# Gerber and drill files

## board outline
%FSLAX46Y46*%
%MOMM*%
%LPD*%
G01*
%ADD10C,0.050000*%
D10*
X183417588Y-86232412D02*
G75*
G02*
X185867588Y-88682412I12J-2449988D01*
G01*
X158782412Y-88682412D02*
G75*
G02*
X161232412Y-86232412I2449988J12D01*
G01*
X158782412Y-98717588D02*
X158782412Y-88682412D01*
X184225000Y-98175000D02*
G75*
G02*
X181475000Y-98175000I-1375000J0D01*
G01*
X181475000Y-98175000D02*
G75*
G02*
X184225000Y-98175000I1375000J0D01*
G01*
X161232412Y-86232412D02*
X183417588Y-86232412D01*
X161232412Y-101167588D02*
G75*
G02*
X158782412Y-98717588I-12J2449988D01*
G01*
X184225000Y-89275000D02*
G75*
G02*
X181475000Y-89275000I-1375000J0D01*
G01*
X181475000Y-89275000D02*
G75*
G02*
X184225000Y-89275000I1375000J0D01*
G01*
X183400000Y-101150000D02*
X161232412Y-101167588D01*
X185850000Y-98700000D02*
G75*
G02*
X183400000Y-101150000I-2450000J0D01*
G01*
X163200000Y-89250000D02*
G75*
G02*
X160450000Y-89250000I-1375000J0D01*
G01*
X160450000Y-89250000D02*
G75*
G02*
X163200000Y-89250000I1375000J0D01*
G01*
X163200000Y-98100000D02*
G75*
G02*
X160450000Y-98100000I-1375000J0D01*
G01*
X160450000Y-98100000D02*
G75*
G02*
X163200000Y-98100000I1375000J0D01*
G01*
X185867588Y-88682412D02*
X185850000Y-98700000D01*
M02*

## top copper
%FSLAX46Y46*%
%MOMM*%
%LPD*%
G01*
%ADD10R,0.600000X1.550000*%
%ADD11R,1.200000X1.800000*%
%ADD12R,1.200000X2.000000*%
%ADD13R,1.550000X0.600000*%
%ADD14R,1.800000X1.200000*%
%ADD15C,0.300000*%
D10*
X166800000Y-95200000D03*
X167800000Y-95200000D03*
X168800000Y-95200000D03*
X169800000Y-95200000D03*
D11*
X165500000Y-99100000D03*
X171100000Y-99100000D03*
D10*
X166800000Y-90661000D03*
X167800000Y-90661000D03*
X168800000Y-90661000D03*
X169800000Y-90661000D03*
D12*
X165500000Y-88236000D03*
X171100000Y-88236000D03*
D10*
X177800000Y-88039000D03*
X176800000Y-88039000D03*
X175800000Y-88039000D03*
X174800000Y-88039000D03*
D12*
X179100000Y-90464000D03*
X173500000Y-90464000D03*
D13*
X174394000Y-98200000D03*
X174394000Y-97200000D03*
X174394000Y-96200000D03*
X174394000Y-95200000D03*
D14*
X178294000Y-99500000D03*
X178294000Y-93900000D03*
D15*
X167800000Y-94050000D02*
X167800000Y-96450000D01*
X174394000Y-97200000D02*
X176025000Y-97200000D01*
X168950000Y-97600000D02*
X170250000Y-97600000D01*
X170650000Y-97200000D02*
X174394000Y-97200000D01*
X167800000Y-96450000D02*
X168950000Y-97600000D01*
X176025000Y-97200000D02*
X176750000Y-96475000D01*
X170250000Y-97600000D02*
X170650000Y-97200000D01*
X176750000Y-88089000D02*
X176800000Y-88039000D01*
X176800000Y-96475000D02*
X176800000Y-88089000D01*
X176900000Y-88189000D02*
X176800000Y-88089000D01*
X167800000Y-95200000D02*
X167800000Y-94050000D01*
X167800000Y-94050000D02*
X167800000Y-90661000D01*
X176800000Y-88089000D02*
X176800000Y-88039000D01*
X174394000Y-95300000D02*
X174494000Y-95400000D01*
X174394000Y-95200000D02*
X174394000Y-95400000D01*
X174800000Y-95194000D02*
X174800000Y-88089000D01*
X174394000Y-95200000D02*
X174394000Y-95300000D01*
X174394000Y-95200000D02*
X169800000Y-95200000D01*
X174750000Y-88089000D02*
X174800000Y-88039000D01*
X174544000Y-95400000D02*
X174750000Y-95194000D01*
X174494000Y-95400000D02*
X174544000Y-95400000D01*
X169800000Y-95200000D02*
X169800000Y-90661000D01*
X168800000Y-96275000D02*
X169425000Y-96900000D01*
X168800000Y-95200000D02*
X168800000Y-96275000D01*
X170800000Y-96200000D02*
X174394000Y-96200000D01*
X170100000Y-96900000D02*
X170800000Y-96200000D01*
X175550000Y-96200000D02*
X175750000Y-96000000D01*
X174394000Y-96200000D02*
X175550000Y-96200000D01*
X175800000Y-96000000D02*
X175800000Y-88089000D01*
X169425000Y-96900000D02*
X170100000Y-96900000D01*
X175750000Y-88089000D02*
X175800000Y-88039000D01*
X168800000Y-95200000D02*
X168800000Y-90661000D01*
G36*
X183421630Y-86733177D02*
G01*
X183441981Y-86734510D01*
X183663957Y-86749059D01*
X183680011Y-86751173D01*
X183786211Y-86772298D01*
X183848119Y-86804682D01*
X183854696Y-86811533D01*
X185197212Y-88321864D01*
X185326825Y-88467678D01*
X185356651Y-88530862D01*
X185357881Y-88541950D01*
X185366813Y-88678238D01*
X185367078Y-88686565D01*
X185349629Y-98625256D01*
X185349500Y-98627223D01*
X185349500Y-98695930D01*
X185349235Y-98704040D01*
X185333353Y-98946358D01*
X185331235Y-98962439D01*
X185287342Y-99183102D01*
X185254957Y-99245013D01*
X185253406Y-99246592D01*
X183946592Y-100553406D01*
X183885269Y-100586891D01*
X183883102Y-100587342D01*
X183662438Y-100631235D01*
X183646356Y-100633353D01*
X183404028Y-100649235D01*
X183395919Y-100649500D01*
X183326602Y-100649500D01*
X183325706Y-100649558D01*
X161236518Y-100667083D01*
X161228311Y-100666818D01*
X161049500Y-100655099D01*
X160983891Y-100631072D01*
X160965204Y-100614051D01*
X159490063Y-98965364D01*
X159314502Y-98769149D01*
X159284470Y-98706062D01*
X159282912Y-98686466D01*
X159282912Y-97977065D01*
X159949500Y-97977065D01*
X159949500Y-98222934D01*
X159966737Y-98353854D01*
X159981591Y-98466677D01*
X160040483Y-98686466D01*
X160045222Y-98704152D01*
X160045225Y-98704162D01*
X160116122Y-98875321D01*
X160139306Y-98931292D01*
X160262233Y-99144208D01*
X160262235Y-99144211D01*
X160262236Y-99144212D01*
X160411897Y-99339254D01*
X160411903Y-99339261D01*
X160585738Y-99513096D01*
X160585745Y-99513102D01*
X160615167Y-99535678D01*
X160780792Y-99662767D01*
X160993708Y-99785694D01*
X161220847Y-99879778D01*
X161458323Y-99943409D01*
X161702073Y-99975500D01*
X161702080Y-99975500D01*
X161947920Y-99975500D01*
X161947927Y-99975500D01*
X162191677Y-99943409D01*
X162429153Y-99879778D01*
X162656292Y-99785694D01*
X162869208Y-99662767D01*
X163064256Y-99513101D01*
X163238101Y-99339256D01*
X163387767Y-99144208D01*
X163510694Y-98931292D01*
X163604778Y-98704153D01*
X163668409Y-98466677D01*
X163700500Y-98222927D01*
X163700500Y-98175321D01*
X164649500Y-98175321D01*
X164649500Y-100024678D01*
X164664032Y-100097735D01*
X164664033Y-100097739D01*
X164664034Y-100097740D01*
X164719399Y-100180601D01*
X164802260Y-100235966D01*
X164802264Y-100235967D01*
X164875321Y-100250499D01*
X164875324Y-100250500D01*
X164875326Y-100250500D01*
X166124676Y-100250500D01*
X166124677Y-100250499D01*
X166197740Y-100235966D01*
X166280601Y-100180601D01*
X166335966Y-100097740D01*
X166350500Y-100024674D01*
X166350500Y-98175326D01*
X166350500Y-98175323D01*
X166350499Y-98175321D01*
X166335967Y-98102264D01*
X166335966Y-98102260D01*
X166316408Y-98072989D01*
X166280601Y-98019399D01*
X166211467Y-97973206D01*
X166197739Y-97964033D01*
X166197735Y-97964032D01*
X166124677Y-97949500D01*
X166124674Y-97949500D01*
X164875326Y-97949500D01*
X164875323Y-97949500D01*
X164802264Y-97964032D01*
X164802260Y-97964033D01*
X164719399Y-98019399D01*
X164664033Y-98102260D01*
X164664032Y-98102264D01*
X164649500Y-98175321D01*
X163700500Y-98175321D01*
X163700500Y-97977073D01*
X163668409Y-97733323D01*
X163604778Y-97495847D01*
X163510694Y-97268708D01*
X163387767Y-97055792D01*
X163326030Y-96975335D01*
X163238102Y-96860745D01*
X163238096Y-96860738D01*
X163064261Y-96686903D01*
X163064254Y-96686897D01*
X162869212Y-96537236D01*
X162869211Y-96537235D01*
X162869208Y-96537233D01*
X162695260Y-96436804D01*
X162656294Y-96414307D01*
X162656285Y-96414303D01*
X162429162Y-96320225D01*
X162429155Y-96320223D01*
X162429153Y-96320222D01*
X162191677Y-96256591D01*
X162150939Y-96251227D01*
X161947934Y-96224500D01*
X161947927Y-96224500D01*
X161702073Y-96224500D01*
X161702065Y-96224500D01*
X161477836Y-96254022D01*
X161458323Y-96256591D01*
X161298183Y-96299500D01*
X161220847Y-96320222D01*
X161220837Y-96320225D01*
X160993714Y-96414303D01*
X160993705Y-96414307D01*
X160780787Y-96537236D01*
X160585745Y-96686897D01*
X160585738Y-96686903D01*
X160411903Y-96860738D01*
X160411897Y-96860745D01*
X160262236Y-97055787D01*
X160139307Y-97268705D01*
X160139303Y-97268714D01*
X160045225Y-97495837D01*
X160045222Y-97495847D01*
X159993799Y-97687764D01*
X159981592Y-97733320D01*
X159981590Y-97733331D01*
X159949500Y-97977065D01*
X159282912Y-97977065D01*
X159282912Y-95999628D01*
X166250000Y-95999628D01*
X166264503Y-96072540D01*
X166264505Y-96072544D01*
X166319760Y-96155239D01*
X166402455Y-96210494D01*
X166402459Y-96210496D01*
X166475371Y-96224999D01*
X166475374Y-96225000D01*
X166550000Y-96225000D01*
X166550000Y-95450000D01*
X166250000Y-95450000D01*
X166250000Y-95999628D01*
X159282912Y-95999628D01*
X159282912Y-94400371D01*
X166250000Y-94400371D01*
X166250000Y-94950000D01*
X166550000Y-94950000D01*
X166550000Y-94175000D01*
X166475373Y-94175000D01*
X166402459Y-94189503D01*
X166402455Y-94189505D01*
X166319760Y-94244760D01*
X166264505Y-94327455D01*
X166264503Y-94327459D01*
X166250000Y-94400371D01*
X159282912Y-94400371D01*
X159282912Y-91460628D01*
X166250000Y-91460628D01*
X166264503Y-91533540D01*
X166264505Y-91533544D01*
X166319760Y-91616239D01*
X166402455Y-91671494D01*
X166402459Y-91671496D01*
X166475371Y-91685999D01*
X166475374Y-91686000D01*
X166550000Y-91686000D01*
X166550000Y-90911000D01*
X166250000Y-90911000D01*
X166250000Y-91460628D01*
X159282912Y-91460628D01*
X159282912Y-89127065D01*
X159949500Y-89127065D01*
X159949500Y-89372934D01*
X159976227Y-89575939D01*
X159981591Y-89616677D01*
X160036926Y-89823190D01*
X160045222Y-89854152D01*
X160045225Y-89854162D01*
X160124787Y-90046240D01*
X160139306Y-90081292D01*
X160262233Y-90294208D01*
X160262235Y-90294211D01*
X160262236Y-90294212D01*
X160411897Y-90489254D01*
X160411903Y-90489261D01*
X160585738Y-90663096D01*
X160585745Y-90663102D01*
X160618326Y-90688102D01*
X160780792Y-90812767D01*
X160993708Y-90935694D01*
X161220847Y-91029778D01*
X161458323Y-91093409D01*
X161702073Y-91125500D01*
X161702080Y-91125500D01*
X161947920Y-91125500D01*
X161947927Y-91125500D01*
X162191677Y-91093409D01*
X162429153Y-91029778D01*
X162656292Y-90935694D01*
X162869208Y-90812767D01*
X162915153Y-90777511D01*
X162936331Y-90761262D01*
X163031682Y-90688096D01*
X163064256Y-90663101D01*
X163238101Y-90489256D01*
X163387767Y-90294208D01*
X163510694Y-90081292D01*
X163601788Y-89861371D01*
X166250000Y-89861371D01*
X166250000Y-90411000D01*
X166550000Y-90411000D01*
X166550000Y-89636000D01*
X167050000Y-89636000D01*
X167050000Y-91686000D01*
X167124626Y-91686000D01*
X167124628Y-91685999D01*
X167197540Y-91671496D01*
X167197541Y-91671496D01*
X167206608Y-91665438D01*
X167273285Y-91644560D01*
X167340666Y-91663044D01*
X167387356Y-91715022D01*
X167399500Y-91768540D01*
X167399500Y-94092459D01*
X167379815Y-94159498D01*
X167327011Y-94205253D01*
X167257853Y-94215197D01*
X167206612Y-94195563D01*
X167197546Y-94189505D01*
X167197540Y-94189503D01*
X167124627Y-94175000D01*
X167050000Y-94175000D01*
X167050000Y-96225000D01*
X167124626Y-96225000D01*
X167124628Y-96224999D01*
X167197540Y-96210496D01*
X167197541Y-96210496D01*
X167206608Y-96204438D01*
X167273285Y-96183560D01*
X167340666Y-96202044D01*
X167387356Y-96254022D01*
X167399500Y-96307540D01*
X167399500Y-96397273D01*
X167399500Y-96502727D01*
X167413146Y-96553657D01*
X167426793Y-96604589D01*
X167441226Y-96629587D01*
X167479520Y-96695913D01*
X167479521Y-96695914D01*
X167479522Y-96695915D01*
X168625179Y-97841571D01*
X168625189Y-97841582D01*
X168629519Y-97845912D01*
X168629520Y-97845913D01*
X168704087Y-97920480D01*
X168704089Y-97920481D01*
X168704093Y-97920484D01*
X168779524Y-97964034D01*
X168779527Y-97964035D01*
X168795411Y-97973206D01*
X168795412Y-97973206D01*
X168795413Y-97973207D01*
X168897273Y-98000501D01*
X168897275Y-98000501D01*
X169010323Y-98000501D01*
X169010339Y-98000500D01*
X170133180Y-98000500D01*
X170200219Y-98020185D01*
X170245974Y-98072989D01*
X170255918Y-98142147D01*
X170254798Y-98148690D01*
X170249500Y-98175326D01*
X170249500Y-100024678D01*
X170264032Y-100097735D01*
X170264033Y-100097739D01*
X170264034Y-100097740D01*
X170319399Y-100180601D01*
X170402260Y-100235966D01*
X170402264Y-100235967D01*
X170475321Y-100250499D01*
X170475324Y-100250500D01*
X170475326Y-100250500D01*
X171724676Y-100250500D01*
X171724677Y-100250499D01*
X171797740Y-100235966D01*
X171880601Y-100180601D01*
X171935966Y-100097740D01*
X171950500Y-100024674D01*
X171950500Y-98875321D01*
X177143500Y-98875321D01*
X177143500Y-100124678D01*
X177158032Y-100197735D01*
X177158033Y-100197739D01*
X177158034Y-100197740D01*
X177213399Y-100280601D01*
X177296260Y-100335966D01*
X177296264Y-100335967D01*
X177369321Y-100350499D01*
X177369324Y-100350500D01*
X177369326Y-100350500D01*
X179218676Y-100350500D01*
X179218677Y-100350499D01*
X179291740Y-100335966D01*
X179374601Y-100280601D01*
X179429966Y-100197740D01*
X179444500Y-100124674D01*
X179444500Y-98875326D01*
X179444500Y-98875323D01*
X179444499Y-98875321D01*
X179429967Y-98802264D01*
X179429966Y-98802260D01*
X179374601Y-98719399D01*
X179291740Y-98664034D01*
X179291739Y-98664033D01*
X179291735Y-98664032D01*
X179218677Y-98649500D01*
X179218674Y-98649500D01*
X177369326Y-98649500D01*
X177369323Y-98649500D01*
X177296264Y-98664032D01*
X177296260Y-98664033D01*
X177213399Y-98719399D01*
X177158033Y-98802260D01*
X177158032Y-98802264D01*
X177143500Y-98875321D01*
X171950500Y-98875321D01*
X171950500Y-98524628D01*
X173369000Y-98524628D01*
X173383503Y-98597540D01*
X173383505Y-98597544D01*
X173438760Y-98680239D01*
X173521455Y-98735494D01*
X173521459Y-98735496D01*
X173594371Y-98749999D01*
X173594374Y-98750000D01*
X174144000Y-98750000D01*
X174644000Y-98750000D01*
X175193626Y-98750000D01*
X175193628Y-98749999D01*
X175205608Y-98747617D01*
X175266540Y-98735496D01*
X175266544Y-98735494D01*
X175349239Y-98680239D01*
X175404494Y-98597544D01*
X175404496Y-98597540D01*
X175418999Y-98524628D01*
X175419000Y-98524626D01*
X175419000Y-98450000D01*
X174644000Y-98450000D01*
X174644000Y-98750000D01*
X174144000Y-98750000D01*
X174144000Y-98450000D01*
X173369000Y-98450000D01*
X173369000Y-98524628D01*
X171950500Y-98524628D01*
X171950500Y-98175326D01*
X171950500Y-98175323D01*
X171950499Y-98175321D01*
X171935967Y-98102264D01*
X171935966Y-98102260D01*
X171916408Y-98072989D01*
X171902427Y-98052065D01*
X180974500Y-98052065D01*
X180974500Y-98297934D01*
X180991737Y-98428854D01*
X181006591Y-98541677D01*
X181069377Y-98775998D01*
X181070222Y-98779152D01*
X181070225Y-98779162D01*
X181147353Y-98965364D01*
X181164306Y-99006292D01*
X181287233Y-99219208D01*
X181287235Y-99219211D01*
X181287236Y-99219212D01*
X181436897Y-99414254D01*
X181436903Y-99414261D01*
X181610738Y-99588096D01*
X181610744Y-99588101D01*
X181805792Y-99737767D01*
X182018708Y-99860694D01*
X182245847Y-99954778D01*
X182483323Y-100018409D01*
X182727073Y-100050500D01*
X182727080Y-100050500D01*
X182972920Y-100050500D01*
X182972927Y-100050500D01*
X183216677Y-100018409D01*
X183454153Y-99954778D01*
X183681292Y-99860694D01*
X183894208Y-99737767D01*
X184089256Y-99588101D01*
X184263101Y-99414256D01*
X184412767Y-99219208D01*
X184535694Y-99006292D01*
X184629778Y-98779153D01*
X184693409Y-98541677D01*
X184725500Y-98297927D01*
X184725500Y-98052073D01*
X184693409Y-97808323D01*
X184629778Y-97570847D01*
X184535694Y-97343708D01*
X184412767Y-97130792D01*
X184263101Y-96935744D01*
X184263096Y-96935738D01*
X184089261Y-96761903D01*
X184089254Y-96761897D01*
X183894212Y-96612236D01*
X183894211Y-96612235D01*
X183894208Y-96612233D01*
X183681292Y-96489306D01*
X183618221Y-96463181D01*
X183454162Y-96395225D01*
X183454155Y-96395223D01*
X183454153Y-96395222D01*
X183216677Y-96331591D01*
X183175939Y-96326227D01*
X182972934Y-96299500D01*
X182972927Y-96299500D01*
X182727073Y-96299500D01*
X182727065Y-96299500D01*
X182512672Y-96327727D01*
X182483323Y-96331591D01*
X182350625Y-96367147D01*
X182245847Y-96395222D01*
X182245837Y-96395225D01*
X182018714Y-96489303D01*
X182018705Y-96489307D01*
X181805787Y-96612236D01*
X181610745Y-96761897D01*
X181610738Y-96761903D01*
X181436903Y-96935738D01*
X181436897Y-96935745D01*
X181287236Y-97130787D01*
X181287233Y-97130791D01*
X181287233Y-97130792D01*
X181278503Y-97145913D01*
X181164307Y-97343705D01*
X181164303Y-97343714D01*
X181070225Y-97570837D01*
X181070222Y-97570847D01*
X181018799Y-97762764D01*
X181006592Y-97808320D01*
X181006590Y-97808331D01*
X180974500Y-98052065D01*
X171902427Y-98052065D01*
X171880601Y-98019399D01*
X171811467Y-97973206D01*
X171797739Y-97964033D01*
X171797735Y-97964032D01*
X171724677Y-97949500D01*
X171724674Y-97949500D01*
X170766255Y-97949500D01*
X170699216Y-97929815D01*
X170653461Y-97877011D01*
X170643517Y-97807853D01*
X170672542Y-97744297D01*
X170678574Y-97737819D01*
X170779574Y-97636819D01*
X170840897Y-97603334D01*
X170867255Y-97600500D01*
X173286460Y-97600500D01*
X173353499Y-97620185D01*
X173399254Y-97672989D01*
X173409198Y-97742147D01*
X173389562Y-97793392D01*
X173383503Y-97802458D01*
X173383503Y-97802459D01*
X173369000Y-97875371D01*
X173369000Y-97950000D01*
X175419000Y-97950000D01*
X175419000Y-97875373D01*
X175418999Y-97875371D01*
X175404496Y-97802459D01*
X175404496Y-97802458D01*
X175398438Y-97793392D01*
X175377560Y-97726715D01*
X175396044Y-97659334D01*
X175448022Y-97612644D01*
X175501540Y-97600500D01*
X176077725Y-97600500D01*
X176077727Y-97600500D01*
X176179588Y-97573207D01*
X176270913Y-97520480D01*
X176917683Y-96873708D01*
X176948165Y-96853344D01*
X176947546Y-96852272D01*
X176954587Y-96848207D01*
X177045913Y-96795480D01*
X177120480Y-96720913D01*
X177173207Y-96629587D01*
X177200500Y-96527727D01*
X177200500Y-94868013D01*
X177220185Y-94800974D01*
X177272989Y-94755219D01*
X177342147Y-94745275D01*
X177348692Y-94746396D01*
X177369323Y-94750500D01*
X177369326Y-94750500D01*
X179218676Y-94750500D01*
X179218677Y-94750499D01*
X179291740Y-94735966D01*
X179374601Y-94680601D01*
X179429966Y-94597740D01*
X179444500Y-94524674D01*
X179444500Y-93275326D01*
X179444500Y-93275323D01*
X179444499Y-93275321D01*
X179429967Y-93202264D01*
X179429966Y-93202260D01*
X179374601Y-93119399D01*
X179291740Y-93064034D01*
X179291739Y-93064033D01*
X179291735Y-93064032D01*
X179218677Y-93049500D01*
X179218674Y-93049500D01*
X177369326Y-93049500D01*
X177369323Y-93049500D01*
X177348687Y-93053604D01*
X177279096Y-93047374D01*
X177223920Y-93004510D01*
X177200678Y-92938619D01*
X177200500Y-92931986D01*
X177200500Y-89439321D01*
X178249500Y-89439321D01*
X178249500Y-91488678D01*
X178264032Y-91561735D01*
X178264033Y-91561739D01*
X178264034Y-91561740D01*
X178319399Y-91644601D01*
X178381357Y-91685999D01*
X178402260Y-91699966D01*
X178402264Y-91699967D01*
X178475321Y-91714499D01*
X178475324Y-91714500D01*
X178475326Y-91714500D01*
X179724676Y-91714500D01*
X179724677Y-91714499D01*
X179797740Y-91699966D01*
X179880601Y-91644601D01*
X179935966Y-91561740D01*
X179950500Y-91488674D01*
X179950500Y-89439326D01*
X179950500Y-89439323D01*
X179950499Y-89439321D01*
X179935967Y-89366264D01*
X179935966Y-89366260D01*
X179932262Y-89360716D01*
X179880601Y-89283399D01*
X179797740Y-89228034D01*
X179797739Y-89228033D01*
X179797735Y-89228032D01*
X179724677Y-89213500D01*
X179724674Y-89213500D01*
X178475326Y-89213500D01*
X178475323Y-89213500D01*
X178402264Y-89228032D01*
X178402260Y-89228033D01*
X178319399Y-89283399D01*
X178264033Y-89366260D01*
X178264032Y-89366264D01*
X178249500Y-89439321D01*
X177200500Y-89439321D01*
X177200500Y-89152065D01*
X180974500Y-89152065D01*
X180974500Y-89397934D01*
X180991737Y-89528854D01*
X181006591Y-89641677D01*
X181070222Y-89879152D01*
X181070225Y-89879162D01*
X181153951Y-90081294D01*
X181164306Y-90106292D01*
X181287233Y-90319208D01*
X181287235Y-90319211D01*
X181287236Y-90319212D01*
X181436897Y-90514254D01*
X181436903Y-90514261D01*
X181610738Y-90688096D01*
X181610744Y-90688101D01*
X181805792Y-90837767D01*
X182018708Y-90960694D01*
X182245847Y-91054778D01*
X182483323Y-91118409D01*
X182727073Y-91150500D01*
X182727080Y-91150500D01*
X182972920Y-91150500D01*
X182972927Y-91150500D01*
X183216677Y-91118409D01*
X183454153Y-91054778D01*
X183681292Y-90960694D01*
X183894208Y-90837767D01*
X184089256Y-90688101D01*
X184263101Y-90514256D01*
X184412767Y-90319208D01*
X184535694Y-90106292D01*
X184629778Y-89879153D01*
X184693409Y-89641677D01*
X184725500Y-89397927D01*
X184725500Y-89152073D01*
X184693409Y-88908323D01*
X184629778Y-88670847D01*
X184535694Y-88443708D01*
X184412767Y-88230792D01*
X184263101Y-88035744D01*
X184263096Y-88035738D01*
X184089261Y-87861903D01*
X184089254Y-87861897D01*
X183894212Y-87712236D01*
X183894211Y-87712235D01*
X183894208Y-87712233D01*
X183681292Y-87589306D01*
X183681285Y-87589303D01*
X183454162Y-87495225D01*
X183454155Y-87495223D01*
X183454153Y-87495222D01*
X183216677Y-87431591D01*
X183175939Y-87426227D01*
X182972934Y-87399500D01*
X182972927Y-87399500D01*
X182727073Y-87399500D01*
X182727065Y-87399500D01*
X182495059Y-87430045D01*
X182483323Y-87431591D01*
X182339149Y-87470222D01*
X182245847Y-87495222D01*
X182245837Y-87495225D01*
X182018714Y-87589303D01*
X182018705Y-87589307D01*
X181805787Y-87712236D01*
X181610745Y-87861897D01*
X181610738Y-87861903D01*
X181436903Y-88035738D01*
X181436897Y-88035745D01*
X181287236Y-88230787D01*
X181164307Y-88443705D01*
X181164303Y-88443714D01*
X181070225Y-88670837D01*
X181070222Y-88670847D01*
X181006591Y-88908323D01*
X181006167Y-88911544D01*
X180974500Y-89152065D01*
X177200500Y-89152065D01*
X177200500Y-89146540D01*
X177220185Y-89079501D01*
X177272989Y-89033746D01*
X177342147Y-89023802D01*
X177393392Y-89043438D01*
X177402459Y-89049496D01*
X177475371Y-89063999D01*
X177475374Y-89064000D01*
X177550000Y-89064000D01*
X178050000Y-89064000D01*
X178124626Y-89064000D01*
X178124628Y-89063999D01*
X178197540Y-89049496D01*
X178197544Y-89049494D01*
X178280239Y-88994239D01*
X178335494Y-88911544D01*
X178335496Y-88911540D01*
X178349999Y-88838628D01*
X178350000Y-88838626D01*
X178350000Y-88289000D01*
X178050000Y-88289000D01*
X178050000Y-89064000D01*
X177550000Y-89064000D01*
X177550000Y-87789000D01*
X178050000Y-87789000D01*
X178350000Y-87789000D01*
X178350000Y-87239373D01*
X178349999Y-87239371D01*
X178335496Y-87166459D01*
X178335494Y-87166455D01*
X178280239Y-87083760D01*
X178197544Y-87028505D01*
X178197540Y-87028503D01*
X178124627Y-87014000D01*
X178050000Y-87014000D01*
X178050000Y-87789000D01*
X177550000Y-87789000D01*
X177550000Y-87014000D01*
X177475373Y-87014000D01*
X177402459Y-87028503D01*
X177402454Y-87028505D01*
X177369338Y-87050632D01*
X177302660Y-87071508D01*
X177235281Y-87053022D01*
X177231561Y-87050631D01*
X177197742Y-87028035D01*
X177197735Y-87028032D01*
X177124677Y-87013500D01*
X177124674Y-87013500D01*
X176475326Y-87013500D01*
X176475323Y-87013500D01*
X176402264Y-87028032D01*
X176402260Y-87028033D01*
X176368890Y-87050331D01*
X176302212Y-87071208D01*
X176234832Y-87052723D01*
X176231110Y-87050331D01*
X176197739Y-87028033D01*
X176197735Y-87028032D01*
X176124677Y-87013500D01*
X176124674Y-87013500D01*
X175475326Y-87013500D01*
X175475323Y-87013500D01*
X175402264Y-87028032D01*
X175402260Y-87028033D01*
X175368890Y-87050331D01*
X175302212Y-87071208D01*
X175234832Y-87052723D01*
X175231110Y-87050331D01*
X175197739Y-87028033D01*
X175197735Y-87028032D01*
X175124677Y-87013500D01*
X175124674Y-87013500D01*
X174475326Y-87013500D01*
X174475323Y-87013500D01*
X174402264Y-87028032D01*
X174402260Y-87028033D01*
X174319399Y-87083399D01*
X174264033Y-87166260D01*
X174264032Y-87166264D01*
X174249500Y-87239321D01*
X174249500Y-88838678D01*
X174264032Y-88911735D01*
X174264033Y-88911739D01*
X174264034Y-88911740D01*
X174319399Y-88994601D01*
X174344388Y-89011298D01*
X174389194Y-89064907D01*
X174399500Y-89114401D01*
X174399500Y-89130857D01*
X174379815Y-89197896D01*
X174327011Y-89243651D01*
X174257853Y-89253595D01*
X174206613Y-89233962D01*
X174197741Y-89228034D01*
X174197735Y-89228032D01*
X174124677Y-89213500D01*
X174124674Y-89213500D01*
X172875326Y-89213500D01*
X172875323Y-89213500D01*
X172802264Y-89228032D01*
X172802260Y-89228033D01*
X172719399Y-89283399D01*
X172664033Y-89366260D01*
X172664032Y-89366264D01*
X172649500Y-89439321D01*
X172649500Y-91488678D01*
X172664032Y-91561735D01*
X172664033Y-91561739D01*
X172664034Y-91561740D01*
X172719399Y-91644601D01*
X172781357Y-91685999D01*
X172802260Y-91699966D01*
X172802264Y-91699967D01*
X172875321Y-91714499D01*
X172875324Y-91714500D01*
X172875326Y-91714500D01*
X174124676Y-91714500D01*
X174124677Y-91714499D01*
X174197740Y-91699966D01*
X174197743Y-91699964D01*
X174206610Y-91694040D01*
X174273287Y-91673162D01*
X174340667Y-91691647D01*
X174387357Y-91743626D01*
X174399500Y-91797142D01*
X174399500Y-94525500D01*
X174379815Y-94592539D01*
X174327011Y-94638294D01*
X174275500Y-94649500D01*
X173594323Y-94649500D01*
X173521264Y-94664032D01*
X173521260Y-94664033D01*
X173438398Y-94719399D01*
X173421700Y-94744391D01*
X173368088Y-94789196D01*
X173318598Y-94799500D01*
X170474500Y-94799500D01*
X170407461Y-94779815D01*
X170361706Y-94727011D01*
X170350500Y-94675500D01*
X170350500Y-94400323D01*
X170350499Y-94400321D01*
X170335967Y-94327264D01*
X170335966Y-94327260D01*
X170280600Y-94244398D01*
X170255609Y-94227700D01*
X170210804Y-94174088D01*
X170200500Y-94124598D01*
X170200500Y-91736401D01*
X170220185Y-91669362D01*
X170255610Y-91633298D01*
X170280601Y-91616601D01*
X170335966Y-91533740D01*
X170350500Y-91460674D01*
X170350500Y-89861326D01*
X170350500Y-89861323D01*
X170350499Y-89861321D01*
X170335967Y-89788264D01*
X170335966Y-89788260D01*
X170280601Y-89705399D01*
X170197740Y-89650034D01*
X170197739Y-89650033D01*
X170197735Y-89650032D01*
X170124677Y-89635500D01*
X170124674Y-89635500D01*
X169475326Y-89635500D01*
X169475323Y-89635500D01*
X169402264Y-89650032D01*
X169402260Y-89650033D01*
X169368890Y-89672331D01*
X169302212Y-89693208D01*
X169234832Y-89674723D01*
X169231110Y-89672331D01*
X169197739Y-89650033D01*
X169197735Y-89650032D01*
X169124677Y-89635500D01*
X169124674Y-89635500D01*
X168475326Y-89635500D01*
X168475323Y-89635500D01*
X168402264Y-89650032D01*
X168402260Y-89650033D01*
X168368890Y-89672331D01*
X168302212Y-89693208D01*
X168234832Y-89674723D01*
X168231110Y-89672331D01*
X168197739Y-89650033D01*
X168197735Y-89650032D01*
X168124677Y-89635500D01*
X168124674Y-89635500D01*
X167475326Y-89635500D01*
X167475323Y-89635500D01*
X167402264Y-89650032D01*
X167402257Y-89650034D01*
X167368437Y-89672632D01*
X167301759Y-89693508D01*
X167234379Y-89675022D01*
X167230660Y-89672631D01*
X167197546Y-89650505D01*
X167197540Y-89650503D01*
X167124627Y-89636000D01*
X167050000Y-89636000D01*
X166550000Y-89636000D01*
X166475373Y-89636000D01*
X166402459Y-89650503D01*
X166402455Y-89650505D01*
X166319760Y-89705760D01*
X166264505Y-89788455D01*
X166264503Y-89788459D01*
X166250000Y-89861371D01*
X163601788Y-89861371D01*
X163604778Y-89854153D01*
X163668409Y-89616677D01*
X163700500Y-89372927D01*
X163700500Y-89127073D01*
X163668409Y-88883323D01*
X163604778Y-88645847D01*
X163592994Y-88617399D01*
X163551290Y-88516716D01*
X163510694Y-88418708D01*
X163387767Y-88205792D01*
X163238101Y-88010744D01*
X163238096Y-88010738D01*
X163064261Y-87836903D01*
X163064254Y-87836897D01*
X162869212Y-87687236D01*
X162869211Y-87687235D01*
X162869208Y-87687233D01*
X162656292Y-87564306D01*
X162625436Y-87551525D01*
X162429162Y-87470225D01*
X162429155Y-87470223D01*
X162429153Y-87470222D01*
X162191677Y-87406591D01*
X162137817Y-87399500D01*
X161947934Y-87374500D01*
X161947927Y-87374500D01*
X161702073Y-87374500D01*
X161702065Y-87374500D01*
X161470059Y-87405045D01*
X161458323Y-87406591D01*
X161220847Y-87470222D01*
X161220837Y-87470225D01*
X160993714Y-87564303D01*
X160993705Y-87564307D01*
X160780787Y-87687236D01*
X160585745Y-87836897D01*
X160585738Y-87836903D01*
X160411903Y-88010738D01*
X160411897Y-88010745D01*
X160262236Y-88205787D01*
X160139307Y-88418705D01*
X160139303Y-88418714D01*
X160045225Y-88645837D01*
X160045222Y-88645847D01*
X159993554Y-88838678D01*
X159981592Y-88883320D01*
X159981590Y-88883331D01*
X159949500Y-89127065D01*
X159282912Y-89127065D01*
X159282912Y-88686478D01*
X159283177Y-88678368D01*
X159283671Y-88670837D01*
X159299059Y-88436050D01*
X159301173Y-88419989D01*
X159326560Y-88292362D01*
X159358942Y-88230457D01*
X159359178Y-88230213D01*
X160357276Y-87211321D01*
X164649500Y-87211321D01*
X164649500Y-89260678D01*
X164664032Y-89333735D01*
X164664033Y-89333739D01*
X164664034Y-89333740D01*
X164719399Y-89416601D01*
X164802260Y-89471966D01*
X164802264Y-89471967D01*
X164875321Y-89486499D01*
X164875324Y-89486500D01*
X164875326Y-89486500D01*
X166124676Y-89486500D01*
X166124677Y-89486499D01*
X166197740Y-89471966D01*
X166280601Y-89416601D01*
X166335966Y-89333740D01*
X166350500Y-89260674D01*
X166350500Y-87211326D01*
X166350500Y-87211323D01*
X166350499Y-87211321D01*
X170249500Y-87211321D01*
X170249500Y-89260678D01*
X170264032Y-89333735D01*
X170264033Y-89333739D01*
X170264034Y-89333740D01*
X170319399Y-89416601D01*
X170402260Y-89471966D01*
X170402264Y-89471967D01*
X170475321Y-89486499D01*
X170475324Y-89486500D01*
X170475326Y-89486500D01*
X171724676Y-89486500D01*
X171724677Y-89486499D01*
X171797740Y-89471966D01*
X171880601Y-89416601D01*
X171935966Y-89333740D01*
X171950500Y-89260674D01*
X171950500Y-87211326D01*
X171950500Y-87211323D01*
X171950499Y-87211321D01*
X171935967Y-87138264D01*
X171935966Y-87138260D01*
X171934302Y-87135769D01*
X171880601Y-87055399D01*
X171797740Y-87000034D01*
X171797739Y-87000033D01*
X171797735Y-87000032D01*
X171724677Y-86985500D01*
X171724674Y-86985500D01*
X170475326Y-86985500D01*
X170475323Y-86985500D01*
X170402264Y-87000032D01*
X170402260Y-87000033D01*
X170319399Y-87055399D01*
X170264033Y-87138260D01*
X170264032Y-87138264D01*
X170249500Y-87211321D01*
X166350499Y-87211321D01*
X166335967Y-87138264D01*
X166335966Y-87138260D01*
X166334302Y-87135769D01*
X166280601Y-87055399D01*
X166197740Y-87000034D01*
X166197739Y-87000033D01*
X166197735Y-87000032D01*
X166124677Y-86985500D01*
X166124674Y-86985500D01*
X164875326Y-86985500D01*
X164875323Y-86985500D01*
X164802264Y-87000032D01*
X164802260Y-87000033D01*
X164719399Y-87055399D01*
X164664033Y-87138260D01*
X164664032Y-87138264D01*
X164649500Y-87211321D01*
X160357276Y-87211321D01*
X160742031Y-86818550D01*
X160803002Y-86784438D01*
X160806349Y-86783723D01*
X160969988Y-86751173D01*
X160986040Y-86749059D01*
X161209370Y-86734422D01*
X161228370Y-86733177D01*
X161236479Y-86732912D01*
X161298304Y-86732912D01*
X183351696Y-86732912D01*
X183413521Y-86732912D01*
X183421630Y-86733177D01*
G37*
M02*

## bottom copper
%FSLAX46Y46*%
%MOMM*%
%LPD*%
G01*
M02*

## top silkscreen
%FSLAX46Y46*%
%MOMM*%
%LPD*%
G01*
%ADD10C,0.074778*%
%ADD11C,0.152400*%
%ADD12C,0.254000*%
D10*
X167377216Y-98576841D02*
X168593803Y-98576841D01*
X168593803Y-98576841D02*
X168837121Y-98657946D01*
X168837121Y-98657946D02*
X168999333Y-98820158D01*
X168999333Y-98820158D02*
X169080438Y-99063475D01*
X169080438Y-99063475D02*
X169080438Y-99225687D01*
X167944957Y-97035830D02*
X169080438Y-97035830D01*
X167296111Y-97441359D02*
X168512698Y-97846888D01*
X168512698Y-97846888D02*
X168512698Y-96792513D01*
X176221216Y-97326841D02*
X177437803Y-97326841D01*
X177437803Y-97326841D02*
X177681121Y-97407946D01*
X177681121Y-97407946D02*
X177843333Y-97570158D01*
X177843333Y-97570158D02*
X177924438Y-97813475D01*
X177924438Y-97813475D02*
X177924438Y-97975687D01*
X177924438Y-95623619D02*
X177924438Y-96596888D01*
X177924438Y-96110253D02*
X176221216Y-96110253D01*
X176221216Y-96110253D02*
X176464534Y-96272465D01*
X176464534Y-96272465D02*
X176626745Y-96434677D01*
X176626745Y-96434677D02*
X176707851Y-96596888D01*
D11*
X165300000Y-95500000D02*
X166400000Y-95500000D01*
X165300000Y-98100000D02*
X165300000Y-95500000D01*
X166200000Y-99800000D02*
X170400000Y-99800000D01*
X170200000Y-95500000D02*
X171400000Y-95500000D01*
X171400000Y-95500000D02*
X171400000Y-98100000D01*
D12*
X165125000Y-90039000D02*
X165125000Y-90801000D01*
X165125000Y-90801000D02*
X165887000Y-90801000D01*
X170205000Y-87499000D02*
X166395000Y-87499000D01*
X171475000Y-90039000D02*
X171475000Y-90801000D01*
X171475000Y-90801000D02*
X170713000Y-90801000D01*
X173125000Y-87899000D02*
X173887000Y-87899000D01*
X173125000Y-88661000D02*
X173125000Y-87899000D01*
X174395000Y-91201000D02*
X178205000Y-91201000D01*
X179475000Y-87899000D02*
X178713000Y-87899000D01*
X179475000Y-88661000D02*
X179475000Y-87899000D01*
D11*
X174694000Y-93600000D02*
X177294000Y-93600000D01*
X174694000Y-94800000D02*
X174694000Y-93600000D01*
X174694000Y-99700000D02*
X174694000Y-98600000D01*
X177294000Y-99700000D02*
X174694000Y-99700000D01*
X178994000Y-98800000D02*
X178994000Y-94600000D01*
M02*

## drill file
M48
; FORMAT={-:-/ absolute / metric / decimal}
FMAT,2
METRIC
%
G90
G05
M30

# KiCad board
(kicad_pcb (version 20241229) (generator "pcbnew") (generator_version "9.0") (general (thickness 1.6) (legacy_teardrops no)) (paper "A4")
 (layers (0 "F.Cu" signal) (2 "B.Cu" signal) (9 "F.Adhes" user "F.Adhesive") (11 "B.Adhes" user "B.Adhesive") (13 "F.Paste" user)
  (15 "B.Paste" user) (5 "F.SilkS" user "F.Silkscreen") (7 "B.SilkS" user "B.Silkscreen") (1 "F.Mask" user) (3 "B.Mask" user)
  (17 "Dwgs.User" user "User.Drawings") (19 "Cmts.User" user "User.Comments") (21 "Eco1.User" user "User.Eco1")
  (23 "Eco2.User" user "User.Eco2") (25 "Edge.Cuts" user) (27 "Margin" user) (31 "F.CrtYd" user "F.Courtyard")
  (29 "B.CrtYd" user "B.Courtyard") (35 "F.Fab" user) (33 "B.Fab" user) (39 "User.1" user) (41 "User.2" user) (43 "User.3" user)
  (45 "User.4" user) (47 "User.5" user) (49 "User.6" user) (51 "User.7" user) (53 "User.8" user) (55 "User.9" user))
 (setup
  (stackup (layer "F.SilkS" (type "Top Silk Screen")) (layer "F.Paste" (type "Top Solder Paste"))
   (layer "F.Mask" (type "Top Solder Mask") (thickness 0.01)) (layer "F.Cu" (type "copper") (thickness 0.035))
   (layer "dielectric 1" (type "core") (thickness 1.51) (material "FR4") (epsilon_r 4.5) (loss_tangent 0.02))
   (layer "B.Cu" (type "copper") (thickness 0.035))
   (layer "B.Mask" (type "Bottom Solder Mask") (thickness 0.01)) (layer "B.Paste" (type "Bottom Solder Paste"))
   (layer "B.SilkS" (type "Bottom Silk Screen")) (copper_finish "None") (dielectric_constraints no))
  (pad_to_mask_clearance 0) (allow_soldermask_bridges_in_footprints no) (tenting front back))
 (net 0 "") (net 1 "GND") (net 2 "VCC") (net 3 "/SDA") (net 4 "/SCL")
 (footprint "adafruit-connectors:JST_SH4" (layer "F.Cu") (at 168.3 97.206)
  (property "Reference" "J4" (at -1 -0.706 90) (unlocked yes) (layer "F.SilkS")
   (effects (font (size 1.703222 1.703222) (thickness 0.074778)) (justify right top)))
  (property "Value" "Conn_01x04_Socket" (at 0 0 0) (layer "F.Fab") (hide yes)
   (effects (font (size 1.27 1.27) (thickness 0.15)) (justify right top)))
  (fp_line (start -3 -1.706) (end -1.9 -1.706) (stroke (width 0.1524) (type solid)) (layer "F.SilkS"))
  (fp_line (start -3 0.894) (end -3 -1.706) (stroke (width 0.1524) (type solid)) (layer "F.SilkS"))
  (fp_line (start -2.1 2.594) (end 2.1 2.594) (stroke (width 0.1524) (type solid)) (layer "F.SilkS"))
  (fp_line (start 1.9 -1.706) (end 3.1 -1.706) (stroke (width 0.1524) (type solid)) (layer "F.SilkS"))
  (fp_line (start 3.1 -1.706) (end 3.1 0.894) (stroke (width 0.1524) (type solid)) (layer "F.SilkS"))
  (pad "1" smd rect (at -1.5 -2.006 90) (size 1.55 0.6) (layers "F.Cu" "F.Mask" "F.Paste") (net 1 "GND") (solder_mask_margin 0.0508)
   (thermal_bridge_angle 0))
  (pad "2" smd rect (at -0.5 -2.006 90) (size 1.55 0.6) (layers "F.Cu" "F.Mask" "F.Paste") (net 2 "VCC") (solder_mask_margin 0.0508)
   (thermal_bridge_angle 0))
  (pad "3" smd rect (at 0.5 -2.006 90) (size 1.55 0.6) (layers "F.Cu" "F.Mask" "F.Paste") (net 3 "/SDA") (solder_mask_margin 0.0508)
   (thermal_bridge_angle 0))
  (pad "4" smd rect (at 1.5 -2.006 90) (size 1.55 0.6) (layers "F.Cu" "F.Mask" "F.Paste") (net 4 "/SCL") (solder_mask_margin 0.0508)
   (thermal_bridge_angle 0))
  (pad "MT1" smd rect (at -2.8 1.894 90) (size 1.8 1.2) (layers "F.Cu" "F.Mask" "F.Paste") (solder_mask_margin 0.0508)
   (thermal_bridge_angle 0))
  (pad "MT2" smd rect (at 2.8 1.894 90) (size 1.8 1.2) (layers "F.Cu" "F.Mask" "F.Paste") (solder_mask_margin 0.0508)
   (thermal_bridge_angle 0)))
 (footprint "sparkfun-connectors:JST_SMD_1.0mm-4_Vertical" (layer "F.Cu") (at 168.3 89.15)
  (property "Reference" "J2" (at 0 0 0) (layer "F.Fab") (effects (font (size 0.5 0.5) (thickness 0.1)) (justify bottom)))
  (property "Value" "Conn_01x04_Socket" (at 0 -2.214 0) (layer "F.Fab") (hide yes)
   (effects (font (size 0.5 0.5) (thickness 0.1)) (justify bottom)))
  (fp_line (start -3.175 0.889) (end -3.175 1.651) (stroke (width 0.254) (type solid)) (layer "F.SilkS"))
  (fp_line (start -3.175 1.651) (end -2.413 1.651) (stroke (width 0.254) (type solid)) (layer "F.SilkS"))
  (fp_line (start 1.905 -1.651) (end -1.905 -1.651) (stroke (width 0.254) (type solid)) (layer "F.SilkS"))
  (fp_line (start 3.175 0.889) (end 3.175 1.651) (stroke (width 0.254) (type solid)) (layer "F.SilkS"))
  (fp_line (start 3.175 1.651) (end 2.413 1.651) (stroke (width 0.254) (type solid)) (layer "F.SilkS"))
  (pad "1" smd rect (at -1.5 1.511) (size 0.6 1.55) (layers "F.Cu" "F.Mask" "F.Paste") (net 1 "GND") (thermal_bridge_angle 0))
  (pad "2" smd rect (at -0.5 1.511) (size 0.6 1.55) (layers "F.Cu" "F.Mask" "F.Paste") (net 2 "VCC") (thermal_bridge_angle 0))
  (pad "3" smd rect (at 0.5 1.511) (size 0.6 1.55) (layers "F.Cu" "F.Mask" "F.Paste") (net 3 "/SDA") (thermal_bridge_angle 0))
  (pad "4" smd rect (at 1.5 1.511) (size 0.6 1.55) (layers "F.Cu" "F.Mask" "F.Paste") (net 4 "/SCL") (thermal_bridge_angle 0))
  (pad "NC1" smd rect (at -2.8 -0.914) (size 1.2 2) (layers "F.Cu" "F.Mask" "F.Paste") (thermal_bridge_angle 0))
  (pad "NC2" smd rect (at 2.8 -0.914) (size 1.2 2) (layers "F.Cu" "F.Mask" "F.Paste") (thermal_bridge_angle 0)))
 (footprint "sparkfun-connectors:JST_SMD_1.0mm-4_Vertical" (layer "F.Cu") (at 176.3 89.55 180)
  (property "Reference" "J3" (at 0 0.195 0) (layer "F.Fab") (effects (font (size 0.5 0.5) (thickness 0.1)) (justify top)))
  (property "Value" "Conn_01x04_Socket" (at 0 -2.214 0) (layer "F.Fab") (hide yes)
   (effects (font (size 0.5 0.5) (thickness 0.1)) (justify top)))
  (fp_line (start 3.175 1.651) (end 2.413 1.651) (stroke (width 0.254) (type solid)) (layer "F.SilkS"))
  (fp_line (start 3.175 0.889) (end 3.175 1.651) (stroke (width 0.254) (type solid)) (layer "F.SilkS"))
  (fp_line (start 1.905 -1.651) (end -1.905 -1.651) (stroke (width 0.254) (type solid)) (layer "F.SilkS"))
  (fp_line (start -3.175 1.651) (end -2.413 1.651) (stroke (width 0.254) (type solid)) (layer "F.SilkS"))
  (fp_line (start -3.175 0.889) (end -3.175 1.651) (stroke (width 0.254) (type solid)) (layer "F.SilkS"))
  (pad "1" smd rect (at -1.5 1.511 180) (size 0.6 1.55) (layers "F.Cu" "F.Mask" "F.Paste") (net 1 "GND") (thermal_bridge_angle 0))
  (pad "2" smd rect (at -0.5 1.511 180) (size 0.6 1.55) (layers "F.Cu" "F.Mask" "F.Paste") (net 2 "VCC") (thermal_bridge_angle 0))
  (pad "3" smd rect (at 0.5 1.511 180) (size 0.6 1.55) (layers "F.Cu" "F.Mask" "F.Paste") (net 3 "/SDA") (thermal_bridge_angle 0))
  (pad "4" smd rect (at 1.5 1.511 180) (size 0.6 1.55) (layers "F.Cu" "F.Mask" "F.Paste") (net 4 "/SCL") (thermal_bridge_angle 0))
  (pad "NC1" smd rect (at -2.8 -0.914 180) (size 1.2 2) (layers "F.Cu" "F.Mask" "F.Paste") (thermal_bridge_angle 0))
  (pad "NC2" smd rect (at 2.8 -0.914 180) (size 1.2 2) (layers "F.Cu" "F.Mask" "F.Paste") (thermal_bridge_angle 0)))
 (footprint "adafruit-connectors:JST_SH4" (layer "F.Cu") (at 176.4 96.7 90)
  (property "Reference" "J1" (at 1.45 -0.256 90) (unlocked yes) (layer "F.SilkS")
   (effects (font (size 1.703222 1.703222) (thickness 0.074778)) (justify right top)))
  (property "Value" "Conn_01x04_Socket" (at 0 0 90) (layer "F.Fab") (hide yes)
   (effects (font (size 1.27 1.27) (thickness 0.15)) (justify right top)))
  (fp_line (start 3.1 -1.706) (end 3.1 0.894) (stroke (width 0.1524) (type solid)) (layer "F.SilkS"))
  (fp_line (start 1.9 -1.706) (end 3.1 -1.706) (stroke (width 0.1524) (type solid)) (layer "F.SilkS"))
  (fp_line (start -3 -1.706) (end -1.9 -1.706) (stroke (width 0.1524) (type solid)) (layer "F.SilkS"))
  (fp_line (start -3 0.894) (end -3 -1.706) (stroke (width 0.1524) (type solid)) (layer "F.SilkS"))
  (fp_line (start -2.1 2.594) (end 2.1 2.594) (stroke (width 0.1524) (type solid)) (layer "F.SilkS"))
  (pad "1" smd rect (at -1.5 -2.006 180) (size 1.55 0.6) (layers "F.Cu" "F.Mask" "F.Paste") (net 1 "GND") (solder_mask_margin 0.0508)
   (thermal_bridge_angle 0))
  (pad "2" smd rect (at -0.5 -2.006 180) (size 1.55 0.6) (layers "F.Cu" "F.Mask" "F.Paste") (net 2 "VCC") (solder_mask_margin 0.0508)
   (thermal_bridge_angle 0))
  (pad "3" smd rect (at 0.5 -2.006 180) (size 1.55 0.6) (layers "F.Cu" "F.Mask" "F.Paste") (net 3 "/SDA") (solder_mask_margin 0.0508)
   (thermal_bridge_angle 0))
  (pad "4" smd rect (at 1.5 -2.006 180) (size 1.55 0.6) (layers "F.Cu" "F.Mask" "F.Paste") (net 4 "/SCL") (solder_mask_margin 0.0508)
   (thermal_bridge_angle 0))
  (pad "MT1" smd rect (at -2.8 1.894 180) (size 1.8 1.2) (layers "F.Cu" "F.Mask" "F.Paste") (solder_mask_margin 0.0508)
   (thermal_bridge_angle 0))
  (pad "MT2" smd rect (at 2.8 1.894 180) (size 1.8 1.2) (layers "F.Cu" "F.Mask" "F.Paste") (solder_mask_margin 0.0508)
   (thermal_bridge_angle 0)))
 (gr_arc (start 183.417588 86.232412) (mid 185.15 86.95) (end 185.867588 88.682412) (stroke (width 0.05) (type default)) (layer "Edge.Cuts"))
 (gr_arc (start 158.782412 88.682412) (mid 159.5 86.95) (end 161.232412 86.232412) (stroke (width 0.05) (type default)) (layer "Edge.Cuts"))
 (gr_line (start 158.782412 98.717588) (end 158.782412 88.682412) (stroke (width 0.05) (type default)) (layer "Edge.Cuts"))
 (gr_circle (center 182.85 98.175) (end 181.475 98.175) (stroke (width 0.05) (type default)) (fill no) (layer "Edge.Cuts"))
 (gr_line (start 161.232412 86.232412) (end 183.417588 86.232412) (stroke (width 0.05) (type default)) (layer "Edge.Cuts"))
 (gr_arc (start 161.232412 101.167588) (mid 159.5 100.45) (end 158.782412 98.717588) (stroke (width 0.05) (type default))
  (layer "Edge.Cuts"))
 (gr_circle (center 182.85 89.275) (end 184.225 89.275) (stroke (width 0.05) (type default)) (fill no) (layer "Edge.Cuts"))
 (gr_line (start 183.4 101.15) (end 161.232412 101.167588) (stroke (width 0.05) (type default)) (layer "Edge.Cuts"))
 (gr_arc (start 185.85 98.7) (mid 185.132412 100.432412) (end 183.4 101.15) (stroke (width 0.05) (type default)) (layer "Edge.Cuts"))
 (gr_circle (center 161.825 89.25) (end 161.825 90.625) (stroke (width 0.05) (type default)) (fill no) (layer "Edge.Cuts"))
 (gr_circle (center 161.825 98.1) (end 163.2 98.1) (stroke (width 0.05) (type default)) (fill no) (layer "Edge.Cuts"))
 (gr_line (start 185.867588 88.682412) (end 185.85 98.7) (stroke (width 0.05) (type default)) (layer "Edge.Cuts"))
 (segment (start 167.8 94.05) (end 167.8 96.45) (width 0.3) (layer "F.Cu") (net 2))
 (segment (start 174.394 97.2) (end 176.025 97.2) (width 0.3) (layer "F.Cu") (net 2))
 (segment (start 168.95 97.6) (end 170.25 97.6) (width 0.3) (layer "F.Cu") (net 2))
 (segment (start 170.65 97.2) (end 174.394 97.2) (width 0.3) (layer "F.Cu") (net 2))
 (segment (start 167.8 96.45) (end 168.95 97.6) (width 0.3) (layer "F.Cu") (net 2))
 (segment (start 176.025 97.2) (end 176.75 96.475) (width 0.3) (layer "F.Cu") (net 2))
 (segment (start 170.25 97.6) (end 170.65 97.2) (width 0.3) (layer "F.Cu") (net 2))
 (segment (start 176.75 88.089) (end 176.8 88.039) (width 0.3) (layer "F.Cu") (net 2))
 (segment (start 176.8 96.475) (end 176.8 88.089) (width 0.3) (layer "F.Cu") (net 2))
 (segment (start 176.9 88.189) (end 176.8 88.089) (width 0.3) (layer "F.Cu") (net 2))
 (segment (start 167.8 95.2) (end 167.8 94.05) (width 0.3) (layer "F.Cu") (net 2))
 (segment (start 167.8 94.05) (end 167.8 90.661) (width 0.3) (layer "F.Cu") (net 2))
 (segment (start 176.8 88.089) (end 176.8 88.039) (width 0.3) (layer "F.Cu") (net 2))
 (segment (start 174.394 95.3) (end 174.494 95.4) (width 0.3) (layer "F.Cu") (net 4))
 (segment (start 174.394 95.2) (end 174.394 95.4) (width 0.3) (layer "F.Cu") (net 4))
 (segment (start 174.8 95.194) (end 174.8 88.089) (width 0.3) (layer "F.Cu") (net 4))
 (segment (start 174.394 95.2) (end 174.394 95.3) (width 0.3) (layer "F.Cu") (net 4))
 (segment (start 174.394 95.2) (end 169.8 95.2) (width 0.3) (layer "F.Cu") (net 4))
 (segment (start 174.75 88.089) (end 174.8 88.039) (width 0.3) (layer "F.Cu") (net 4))
 (segment (start 174.544 95.4) (end 174.75 95.194) (width 0.3) (layer "F.Cu") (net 4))
 (segment (start 174.494 95.4) (end 174.544 95.4) (width 0.3) (layer "F.Cu") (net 4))
 (segment (start 169.8 95.2) (end 169.8 90.661) (width 0.3) (layer "F.Cu") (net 4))
 (segment (start 168.8 96.275) (end 169.425 96.9) (width 0.3) (layer "F.Cu") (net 3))
 (segment (start 168.8 95.2) (end 168.8 96.275) (width 0.3) (layer "F.Cu") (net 3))
 (segment (start 170.8 96.2) (end 174.394 96.2) (width 0.3) (layer "F.Cu") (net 3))
 (segment (start 170.1 96.9) (end 170.8 96.2) (width 0.3) (layer "F.Cu") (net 3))
 (segment (start 175.55 96.2) (end 175.75 96) (width 0.3) (layer "F.Cu") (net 3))
 (segment (start 174.394 96.2) (end 175.55 96.2) (width 0.3) (layer "F.Cu") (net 3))
 (segment (start 175.8 96) (end 175.8 88.089) (width 0.3) (layer "F.Cu") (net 3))
 (segment (start 169.425 96.9) (end 170.1 96.9) (width 0.3) (layer "F.Cu") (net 3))
 (segment (start 175.75 88.089) (end 175.8 88.039) (width 0.3) (layer "F.Cu") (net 3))
 (segment (start 168.8 95.2) (end 168.8 90.661) (width 0.3) (layer "F.Cu") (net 3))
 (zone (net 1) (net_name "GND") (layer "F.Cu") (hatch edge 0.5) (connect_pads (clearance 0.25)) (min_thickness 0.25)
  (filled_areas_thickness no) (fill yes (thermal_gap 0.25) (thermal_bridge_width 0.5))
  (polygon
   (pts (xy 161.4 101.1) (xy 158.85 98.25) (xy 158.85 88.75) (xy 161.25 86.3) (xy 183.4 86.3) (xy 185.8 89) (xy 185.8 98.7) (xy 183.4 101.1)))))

